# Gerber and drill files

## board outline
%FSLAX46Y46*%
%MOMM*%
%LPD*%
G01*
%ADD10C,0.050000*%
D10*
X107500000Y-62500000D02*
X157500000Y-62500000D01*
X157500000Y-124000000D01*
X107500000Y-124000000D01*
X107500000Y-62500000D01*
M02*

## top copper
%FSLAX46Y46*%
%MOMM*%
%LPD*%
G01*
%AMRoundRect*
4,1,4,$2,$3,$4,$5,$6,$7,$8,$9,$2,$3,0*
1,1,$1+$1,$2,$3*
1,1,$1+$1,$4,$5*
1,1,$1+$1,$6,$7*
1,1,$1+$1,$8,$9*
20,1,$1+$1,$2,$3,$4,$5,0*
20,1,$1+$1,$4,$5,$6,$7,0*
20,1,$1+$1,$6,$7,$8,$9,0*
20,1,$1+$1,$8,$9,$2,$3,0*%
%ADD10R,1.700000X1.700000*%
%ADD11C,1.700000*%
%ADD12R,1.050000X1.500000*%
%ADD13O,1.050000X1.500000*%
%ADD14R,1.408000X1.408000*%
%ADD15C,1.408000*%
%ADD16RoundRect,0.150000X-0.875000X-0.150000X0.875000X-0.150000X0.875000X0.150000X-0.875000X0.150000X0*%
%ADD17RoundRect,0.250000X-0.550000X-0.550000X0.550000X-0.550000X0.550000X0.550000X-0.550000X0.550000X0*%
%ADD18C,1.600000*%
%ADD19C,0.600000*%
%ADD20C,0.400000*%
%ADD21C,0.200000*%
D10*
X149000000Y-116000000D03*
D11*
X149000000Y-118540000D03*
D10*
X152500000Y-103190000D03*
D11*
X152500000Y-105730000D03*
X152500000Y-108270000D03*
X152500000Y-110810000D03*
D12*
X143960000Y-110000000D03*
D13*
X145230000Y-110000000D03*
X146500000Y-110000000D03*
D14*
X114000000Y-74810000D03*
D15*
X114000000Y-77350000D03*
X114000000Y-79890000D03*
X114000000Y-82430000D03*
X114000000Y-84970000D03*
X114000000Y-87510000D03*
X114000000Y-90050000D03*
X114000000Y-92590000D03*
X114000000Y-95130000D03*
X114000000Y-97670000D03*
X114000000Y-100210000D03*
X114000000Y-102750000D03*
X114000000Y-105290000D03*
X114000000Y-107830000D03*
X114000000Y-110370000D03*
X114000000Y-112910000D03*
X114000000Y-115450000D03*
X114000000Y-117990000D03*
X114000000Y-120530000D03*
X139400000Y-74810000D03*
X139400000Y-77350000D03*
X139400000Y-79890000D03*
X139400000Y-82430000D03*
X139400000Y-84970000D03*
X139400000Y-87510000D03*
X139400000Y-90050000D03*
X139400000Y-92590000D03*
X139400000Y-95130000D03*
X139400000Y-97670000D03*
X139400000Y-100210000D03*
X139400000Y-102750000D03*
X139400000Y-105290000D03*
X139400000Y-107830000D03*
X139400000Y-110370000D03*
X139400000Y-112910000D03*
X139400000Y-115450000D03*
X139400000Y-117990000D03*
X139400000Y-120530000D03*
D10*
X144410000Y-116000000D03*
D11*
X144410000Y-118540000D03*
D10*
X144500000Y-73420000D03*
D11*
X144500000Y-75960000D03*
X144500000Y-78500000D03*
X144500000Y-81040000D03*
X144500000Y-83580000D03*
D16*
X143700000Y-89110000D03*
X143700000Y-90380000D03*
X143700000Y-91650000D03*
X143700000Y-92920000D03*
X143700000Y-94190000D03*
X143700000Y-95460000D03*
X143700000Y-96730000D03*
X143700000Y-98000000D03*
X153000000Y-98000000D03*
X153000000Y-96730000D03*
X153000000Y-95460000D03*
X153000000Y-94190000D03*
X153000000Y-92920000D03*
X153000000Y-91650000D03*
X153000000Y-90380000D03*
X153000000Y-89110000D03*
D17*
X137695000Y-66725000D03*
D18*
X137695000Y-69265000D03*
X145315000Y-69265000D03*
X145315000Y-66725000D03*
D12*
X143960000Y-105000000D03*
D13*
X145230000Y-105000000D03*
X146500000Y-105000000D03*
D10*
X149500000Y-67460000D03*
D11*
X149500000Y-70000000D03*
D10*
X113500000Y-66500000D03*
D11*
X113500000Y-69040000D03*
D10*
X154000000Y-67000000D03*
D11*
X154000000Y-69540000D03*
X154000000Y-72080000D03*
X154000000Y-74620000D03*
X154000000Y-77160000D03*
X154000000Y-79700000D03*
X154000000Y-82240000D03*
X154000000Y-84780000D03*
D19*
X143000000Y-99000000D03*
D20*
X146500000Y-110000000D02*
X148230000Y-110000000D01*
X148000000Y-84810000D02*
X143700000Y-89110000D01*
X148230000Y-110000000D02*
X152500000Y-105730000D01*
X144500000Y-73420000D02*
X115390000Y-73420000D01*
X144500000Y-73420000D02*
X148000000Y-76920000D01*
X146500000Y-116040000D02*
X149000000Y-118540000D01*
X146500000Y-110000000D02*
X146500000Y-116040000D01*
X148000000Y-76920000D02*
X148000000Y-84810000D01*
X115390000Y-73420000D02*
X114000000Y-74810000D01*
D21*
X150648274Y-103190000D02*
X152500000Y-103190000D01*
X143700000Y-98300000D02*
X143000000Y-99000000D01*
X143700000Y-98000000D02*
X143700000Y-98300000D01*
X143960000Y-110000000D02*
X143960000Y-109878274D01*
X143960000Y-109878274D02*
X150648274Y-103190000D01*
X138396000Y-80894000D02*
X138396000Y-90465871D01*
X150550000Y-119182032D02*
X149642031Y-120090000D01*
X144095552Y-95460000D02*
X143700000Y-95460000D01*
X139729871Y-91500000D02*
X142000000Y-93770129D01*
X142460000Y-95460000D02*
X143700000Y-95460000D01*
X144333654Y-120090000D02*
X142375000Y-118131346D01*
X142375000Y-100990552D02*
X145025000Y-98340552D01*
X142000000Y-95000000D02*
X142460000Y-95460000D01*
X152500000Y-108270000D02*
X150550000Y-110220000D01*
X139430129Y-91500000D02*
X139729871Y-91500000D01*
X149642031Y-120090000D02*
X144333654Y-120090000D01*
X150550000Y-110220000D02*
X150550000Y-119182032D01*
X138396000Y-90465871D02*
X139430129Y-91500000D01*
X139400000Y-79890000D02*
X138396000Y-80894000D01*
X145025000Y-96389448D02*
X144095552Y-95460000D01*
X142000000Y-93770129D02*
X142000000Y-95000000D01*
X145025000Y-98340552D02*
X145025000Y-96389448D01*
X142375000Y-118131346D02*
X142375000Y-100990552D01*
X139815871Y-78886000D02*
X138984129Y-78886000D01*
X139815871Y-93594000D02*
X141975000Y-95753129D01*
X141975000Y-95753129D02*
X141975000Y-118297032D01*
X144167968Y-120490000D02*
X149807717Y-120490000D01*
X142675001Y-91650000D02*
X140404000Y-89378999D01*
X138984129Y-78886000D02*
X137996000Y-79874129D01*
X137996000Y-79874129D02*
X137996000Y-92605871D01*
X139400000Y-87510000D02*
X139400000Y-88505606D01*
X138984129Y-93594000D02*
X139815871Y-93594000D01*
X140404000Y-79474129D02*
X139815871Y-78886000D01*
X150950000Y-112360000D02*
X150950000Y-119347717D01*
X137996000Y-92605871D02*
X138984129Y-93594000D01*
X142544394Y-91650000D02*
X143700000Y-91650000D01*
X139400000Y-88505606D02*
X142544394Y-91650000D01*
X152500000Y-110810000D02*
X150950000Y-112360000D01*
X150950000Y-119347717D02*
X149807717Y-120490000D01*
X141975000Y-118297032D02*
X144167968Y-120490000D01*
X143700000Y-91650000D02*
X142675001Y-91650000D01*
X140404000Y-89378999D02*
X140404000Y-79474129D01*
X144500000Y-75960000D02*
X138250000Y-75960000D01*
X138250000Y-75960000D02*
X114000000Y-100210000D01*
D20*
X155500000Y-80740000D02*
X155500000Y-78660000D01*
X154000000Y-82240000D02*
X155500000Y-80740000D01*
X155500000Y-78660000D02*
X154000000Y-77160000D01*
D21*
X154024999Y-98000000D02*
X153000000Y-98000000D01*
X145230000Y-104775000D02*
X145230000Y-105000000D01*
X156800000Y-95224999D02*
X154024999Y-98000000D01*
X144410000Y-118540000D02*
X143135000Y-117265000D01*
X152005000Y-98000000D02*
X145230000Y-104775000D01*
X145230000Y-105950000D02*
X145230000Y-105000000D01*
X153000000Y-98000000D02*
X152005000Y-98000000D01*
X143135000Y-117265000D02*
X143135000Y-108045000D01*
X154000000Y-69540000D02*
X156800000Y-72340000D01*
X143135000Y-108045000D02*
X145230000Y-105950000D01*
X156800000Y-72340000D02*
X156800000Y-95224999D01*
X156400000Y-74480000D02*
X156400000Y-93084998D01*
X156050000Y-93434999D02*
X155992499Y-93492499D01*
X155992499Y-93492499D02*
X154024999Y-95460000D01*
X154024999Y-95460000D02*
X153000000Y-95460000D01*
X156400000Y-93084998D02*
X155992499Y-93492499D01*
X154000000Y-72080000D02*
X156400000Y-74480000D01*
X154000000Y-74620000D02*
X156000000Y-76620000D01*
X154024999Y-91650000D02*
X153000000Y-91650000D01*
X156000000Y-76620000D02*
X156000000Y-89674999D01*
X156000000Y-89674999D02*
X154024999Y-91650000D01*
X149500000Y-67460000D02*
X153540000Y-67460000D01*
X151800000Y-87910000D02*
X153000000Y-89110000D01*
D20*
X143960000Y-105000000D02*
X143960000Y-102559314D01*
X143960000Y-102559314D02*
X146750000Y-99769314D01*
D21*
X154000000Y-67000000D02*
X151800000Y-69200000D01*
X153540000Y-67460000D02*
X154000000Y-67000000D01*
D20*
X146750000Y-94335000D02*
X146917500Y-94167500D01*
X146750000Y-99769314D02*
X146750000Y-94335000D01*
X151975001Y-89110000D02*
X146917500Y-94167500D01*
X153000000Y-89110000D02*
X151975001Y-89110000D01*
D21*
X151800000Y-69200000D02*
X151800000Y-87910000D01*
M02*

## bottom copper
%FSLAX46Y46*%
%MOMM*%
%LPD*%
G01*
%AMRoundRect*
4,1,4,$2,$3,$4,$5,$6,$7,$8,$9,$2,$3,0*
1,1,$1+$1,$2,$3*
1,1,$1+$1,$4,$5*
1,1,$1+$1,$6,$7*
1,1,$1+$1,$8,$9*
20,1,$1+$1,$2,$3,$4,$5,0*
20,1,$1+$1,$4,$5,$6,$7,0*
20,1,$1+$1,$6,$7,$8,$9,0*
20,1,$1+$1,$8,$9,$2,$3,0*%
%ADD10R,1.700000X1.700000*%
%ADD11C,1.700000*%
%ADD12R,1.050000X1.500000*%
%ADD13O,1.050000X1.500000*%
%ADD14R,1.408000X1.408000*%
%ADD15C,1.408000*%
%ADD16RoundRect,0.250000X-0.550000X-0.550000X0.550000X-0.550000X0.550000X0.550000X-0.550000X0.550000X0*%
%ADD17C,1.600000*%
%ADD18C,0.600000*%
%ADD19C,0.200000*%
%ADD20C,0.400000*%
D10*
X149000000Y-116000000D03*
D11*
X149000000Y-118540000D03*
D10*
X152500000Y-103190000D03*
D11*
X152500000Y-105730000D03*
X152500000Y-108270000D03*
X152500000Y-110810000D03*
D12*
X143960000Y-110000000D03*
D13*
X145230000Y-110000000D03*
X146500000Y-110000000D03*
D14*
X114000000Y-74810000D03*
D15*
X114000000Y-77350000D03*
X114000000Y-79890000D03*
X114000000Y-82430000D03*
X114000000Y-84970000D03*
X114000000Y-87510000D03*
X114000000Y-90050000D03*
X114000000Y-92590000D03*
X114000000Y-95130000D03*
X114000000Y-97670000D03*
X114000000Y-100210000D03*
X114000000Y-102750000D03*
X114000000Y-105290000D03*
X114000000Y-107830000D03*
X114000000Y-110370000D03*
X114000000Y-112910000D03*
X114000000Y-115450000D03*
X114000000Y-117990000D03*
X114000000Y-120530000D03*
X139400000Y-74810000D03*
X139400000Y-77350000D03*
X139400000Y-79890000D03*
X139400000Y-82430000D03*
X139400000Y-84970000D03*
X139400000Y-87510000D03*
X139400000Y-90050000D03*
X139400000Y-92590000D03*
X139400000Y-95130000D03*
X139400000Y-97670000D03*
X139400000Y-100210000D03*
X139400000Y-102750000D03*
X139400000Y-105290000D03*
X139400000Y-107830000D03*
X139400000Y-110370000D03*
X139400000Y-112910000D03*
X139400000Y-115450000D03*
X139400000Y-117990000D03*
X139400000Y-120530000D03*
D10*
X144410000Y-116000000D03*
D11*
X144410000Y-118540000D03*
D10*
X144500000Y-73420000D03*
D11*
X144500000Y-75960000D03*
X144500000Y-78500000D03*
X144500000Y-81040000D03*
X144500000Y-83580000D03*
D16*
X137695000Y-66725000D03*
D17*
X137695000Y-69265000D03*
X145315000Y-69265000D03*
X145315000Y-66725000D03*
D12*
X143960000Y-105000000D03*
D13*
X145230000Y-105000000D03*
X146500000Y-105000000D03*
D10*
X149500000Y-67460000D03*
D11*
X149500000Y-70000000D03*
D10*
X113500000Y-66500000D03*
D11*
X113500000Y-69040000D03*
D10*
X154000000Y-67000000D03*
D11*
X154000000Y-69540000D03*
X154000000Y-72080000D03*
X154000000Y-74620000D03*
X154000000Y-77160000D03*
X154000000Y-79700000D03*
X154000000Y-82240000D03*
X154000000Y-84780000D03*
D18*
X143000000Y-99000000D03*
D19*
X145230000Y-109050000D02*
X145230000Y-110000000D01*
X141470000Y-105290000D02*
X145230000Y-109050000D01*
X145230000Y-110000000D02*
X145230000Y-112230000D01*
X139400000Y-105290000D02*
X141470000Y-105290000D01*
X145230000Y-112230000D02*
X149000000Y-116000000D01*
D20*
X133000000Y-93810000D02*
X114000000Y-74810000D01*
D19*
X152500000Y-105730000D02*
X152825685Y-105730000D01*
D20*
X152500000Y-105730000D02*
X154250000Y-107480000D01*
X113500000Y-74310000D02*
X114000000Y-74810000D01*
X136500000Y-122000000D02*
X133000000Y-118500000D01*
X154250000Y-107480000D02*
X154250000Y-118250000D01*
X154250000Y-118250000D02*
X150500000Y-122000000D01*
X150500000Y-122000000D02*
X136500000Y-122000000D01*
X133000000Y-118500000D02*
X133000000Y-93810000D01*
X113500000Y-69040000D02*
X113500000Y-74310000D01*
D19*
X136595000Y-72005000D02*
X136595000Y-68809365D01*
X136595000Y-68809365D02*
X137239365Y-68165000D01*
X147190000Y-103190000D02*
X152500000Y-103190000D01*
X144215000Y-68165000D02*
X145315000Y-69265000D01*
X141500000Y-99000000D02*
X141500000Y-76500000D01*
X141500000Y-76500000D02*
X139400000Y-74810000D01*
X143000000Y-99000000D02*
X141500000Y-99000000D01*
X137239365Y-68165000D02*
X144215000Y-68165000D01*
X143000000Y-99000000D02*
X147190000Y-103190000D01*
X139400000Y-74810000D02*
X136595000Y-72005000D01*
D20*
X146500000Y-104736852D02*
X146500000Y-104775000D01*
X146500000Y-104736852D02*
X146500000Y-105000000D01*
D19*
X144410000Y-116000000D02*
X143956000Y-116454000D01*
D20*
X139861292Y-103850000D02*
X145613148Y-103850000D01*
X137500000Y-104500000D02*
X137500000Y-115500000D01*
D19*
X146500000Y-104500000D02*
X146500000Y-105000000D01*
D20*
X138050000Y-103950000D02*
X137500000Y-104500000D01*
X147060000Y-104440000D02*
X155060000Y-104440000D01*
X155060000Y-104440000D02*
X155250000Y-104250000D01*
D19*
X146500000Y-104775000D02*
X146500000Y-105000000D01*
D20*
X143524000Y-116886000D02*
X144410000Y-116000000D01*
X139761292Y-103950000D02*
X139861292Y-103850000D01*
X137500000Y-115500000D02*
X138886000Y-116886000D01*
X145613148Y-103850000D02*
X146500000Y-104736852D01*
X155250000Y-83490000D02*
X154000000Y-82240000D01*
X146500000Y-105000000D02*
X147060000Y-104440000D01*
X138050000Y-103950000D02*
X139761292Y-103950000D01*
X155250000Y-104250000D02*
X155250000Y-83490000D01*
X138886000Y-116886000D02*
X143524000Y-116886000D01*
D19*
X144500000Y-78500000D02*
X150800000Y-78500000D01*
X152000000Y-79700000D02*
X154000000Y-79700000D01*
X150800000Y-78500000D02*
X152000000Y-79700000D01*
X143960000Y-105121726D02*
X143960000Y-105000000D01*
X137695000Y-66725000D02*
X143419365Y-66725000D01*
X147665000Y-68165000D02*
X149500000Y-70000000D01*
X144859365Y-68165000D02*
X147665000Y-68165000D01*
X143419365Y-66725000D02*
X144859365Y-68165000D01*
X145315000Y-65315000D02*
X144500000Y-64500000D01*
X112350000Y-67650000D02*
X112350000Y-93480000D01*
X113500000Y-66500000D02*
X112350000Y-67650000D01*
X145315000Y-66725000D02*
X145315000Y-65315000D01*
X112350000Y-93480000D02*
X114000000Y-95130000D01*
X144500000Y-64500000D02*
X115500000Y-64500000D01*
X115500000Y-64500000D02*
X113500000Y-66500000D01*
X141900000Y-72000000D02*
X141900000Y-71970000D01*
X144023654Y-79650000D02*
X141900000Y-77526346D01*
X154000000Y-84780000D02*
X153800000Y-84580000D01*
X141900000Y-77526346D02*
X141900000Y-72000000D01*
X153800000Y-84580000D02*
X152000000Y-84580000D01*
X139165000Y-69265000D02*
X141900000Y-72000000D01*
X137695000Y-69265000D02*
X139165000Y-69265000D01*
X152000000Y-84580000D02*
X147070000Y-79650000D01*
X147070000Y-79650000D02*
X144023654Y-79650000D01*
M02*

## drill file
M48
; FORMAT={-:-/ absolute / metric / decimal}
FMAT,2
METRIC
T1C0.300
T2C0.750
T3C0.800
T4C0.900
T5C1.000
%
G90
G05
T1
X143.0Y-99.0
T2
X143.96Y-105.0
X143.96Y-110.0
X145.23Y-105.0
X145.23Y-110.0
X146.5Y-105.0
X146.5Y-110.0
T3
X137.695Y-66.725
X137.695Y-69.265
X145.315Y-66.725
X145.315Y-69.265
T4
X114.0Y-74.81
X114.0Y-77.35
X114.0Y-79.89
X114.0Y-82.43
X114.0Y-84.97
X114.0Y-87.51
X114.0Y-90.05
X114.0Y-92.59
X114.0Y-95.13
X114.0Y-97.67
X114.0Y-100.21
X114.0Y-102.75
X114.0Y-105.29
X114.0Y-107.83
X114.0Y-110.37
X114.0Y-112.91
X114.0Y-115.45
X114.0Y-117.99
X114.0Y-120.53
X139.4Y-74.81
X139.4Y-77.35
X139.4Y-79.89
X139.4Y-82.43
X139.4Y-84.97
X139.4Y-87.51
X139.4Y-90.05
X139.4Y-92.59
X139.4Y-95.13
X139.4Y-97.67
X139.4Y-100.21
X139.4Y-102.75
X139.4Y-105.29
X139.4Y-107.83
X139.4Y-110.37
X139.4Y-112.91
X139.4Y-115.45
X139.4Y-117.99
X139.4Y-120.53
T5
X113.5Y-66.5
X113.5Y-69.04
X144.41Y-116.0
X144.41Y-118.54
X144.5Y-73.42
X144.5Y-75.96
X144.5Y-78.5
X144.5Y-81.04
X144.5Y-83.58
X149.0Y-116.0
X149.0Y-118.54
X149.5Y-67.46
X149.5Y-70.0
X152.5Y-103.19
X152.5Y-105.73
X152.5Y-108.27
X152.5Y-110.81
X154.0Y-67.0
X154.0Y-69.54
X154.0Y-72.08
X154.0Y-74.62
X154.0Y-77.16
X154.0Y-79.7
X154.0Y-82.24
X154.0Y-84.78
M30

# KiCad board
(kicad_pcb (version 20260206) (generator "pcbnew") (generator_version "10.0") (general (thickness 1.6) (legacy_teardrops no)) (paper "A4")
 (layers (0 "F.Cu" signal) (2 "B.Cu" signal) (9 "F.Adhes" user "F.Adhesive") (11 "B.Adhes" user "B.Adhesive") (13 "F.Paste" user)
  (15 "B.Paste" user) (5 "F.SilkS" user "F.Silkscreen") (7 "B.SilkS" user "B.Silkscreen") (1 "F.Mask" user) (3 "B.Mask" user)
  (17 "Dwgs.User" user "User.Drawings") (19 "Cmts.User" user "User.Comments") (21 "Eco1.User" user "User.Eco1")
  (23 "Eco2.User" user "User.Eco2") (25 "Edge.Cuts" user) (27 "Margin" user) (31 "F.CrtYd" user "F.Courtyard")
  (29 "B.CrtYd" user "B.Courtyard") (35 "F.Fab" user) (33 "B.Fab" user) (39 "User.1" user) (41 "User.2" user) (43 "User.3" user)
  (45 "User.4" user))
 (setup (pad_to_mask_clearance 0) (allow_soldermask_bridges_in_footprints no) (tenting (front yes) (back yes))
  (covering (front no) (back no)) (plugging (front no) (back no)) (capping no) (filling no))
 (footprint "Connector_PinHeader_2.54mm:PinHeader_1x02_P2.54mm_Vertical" (layer "F.Cu") (at 149 116)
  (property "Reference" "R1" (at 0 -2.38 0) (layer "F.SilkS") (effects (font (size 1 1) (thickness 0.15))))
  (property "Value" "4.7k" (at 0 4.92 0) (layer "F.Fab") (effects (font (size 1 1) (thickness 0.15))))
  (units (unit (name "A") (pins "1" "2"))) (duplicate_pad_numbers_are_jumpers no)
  (pad "1" thru_hole rect (at 0 0) (size 1.7 1.7) (drill 1) (layers "*.Cu" "*.Mask") (remove_unused_layers no) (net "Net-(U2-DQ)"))
  (pad "2" thru_hole circle (at 0 2.54) (size 1.7 1.7) (drill 1) (layers "*.Cu" "*.Mask") (remove_unused_layers no) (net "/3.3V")))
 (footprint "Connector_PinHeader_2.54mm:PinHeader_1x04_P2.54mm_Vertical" (layer "F.Cu") (at 152.5 103.19)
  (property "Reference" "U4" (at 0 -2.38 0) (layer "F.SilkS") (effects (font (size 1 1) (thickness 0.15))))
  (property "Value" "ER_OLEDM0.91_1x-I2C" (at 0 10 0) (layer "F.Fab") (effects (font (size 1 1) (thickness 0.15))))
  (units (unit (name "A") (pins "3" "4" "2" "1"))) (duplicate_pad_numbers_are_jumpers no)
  (pad "1" thru_hole rect (at 0 0) (size 1.7 1.7) (drill 1) (layers "*.Cu" "*.Mask") (remove_unused_layers no) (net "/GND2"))
  (pad "2" thru_hole circle (at 0 2.54) (size 1.7 1.7) (drill 1) (layers "*.Cu" "*.Mask") (remove_unused_layers no) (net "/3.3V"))
  (pad "3" thru_hole circle (at 0 5.08) (size 1.7 1.7) (drill 1) (layers "*.Cu" "*.Mask") (remove_unused_layers no) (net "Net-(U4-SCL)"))
  (pad "4" thru_hole circle (at 0 7.62) (size 1.7 1.7) (drill 1) (layers "*.Cu" "*.Mask") (remove_unused_layers no) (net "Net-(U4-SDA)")))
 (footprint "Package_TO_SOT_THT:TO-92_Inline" (layer "F.Cu") (at 143.96 110)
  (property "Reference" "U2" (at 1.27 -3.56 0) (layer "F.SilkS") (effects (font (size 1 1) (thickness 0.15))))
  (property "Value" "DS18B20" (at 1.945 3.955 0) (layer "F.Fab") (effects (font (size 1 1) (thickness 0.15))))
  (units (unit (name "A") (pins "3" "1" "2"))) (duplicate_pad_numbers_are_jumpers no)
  (pad "1" thru_hole rect (at 0 0) (size 1.05 1.5) (drill 0.75) (layers "*.Cu" "*.Mask") (remove_unused_layers no) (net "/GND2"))
  (pad "2" thru_hole oval (at 1.27 0) (size 1.05 1.5) (drill 0.75) (layers "*.Cu" "*.Mask") (remove_unused_layers no) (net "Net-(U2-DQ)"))
  (pad "3" thru_hole oval (at 2.54 0) (size 1.05 1.5) (drill 0.75) (layers "*.Cu" "*.Mask") (remove_unused_layers no) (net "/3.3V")))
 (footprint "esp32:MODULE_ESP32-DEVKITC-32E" (layer "F.Cu") (at 126.7 97.645)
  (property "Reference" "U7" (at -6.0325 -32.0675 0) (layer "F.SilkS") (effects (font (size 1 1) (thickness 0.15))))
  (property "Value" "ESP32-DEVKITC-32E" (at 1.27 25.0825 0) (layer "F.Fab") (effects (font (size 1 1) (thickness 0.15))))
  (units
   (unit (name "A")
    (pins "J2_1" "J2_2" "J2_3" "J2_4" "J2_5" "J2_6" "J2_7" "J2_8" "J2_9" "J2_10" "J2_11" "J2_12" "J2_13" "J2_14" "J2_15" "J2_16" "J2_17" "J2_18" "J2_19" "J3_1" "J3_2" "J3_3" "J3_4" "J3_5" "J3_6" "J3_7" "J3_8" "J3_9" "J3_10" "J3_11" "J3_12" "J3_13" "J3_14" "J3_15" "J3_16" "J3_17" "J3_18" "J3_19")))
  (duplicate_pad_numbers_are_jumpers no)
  (pad "J2_1" thru_hole rect (at -12.7 -22.835) (size 1.408 1.408) (drill 0.9) (layers "*.Cu" "*.Mask") (remove_unused_layers no)
   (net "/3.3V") (solder_mask_margin 0.102))
  (pad "J2_2" thru_hole circle (at -12.7 -20.295) (size 1.408 1.408) (drill 0.9) (layers "*.Cu" "*.Mask") (remove_unused_layers no)
   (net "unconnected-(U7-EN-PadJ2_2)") (solder_mask_margin 0.102))
  (pad "J2_3" thru_hole circle (at -12.7 -17.755) (size 1.408 1.408) (drill 0.9) (layers "*.Cu" "*.Mask") (remove_unused_layers no)
   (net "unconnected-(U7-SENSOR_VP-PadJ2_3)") (solder_mask_margin 0.102))
  (pad "J2_4" thru_hole circle (at -12.7 -15.215) (size 1.408 1.408) (drill 0.9) (layers "*.Cu" "*.Mask") (remove_unused_layers no)
   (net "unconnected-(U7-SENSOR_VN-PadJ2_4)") (solder_mask_margin 0.102))
  (pad "J2_5" thru_hole circle (at -12.7 -12.675) (size 1.408 1.408) (drill 0.9) (layers "*.Cu" "*.Mask") (remove_unused_layers no)
   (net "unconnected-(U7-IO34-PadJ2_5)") (solder_mask_margin 0.102))
  (pad "J2_6" thru_hole circle (at -12.7 -10.135) (size 1.408 1.408) (drill 0.9) (layers "*.Cu" "*.Mask") (remove_unused_layers no)
   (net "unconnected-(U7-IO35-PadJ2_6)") (solder_mask_margin 0.102))
  (pad "J2_7" thru_hole circle (at -12.7 -7.595) (size 1.408 1.408) (drill 0.9) (layers "*.Cu" "*.Mask") (remove_unused_layers no)
   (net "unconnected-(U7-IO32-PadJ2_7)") (solder_mask_margin 0.102))
  (pad "J2_8" thru_hole circle (at -12.7 -5.055) (size 1.408 1.408) (drill 0.9) (layers "*.Cu" "*.Mask") (remove_unused_layers no)
   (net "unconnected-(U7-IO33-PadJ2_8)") (solder_mask_margin 0.102))
  (pad "J2_9" thru_hole circle (at -12.7 -2.515) (size 1.408 1.408) (drill 0.9) (layers "*.Cu" "*.Mask") (remove_unused_layers no)
   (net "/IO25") (solder_mask_margin 0.102))
  (pad "J2_10" thru_hole circle (at -12.7 0.025) (size 1.408 1.408) (drill 0.9) (layers "*.Cu" "*.Mask") (remove_unused_layers no)
   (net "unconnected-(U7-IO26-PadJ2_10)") (solder_mask_margin 0.102))
  (pad "J2_11" thru_hole circle (at -12.7 2.565) (size 1.408 1.408) (drill 0.9) (layers "*.Cu" "*.Mask") (remove_unused_layers no)
   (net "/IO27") (solder_mask_margin 0.102))
  (pad "J2_12" thru_hole circle (at -12.7 5.105) (size 1.408 1.408) (drill 0.9) (layers "*.Cu" "*.Mask") (remove_unused_layers no)
   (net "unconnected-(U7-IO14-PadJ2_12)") (solder_mask_margin 0.102))
  (pad "J2_13" thru_hole circle (at -12.7 7.645) (size 1.408 1.408) (drill 0.9) (layers "*.Cu" "*.Mask") (remove_unused_layers no)
   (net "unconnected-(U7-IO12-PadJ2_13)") (solder_mask_margin 0.102))
  (pad "J2_14" thru_hole circle (at -12.7 10.185) (size 1.408 1.408) (drill 0.9) (layers "*.Cu" "*.Mask") (remove_unused_layers no)
   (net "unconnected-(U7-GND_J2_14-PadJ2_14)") (solder_mask_margin 0.102))
  (pad "J2_15" thru_hole circle (at -12.7 12.725) (size 1.408 1.408) (drill 0.9) (layers "*.Cu" "*.Mask") (remove_unused_layers no)
   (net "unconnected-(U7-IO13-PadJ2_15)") (solder_mask_margin 0.102))
  (pad "J2_16" thru_hole circle (at -12.7 15.265) (size 1.408 1.408) (drill 0.9) (layers "*.Cu" "*.Mask") (remove_unused_layers no)
   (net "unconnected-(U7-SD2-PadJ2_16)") (solder_mask_margin 0.102))
  (pad "J2_17" thru_hole circle (at -12.7 17.805) (size 1.408 1.408) (drill 0.9) (layers "*.Cu" "*.Mask") (remove_unused_layers no)
   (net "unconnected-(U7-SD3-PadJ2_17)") (solder_mask_margin 0.102))
  (pad "J2_18" thru_hole circle (at -12.7 20.345) (size 1.408 1.408) (drill 0.9) (layers "*.Cu" "*.Mask") (remove_unused_layers no)
   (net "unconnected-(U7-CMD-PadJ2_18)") (solder_mask_margin 0.102))
  (pad "J2_19" thru_hole circle (at -12.7 22.885) (size 1.408 1.408) (drill 0.9) (layers "*.Cu" "*.Mask") (remove_unused_layers no)
   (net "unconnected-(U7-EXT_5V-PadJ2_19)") (solder_mask_margin 0.102))
  (pad "J3_1" thru_hole circle (at 12.7 -22.835) (size 1.408 1.408) (drill 0.9) (layers "*.Cu" "*.Mask") (remove_unused_layers no)
   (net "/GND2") (solder_mask_margin 0.102))
  (pad "J3_2" thru_hole circle (at 12.7 -20.295) (size 1.408 1.408) (drill 0.9) (layers "*.Cu" "*.Mask") (remove_unused_layers no)
   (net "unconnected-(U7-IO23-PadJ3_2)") (solder_mask_margin 0.102))
  (pad "J3_3" thru_hole circle (at 12.7 -17.755) (size 1.408 1.408) (drill 0.9) (layers "*.Cu" "*.Mask") (remove_unused_layers no)
   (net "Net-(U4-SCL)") (solder_mask_margin 0.102))
  (pad "J3_4" thru_hole circle (at 12.7 -15.215) (size 1.408 1.408) (drill 0.9) (layers "*.Cu" "*.Mask") (remove_unused_layers no)
   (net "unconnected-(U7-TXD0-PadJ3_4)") (solder_mask_margin 0.102))
  (pad "J3_5" thru_hole circle (at 12.7 -12.675) (size 1.408 1.408) (drill 0.9) (layers "*.Cu" "*.Mask") (remove_unused_layers no)
   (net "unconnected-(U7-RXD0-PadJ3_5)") (solder_mask_margin 0.102))
  (pad "J3_6" thru_hole circle (at 12.7 -10.135) (size 1.408 1.408) (drill 0.9) (layers "*.Cu" "*.Mask") (remove_unused_layers no)
   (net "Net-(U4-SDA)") (solder_mask_margin 0.102))
  (pad "J3_7" thru_hole circle (at 12.7 -7.595) (size 1.408 1.408) (drill 0.9) (layers "*.Cu" "*.Mask") (remove_unused_layers no)
   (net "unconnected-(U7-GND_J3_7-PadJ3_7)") (solder_mask_margin 0.102))
  (pad "J3_8" thru_hole circle (at 12.7 -5.055) (size 1.408 1.408) (drill 0.9) (layers "*.Cu" "*.Mask") (remove_unused_layers no)
   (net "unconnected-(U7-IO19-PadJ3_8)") (solder_mask_margin 0.102))
  (pad "J3_9" thru_hole circle (at 12.7 -2.515) (size 1.408 1.408) (drill 0.9) (layers "*.Cu" "*.Mask") (remove_unused_layers no)
   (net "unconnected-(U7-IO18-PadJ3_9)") (solder_mask_margin 0.102))
  (pad "J3_10" thru_hole circle (at 12.7 0.025) (size 1.408 1.408) (drill 0.9) (layers "*.Cu" "*.Mask") (remove_unused_layers no)
   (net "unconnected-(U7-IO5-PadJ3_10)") (solder_mask_margin 0.102))
  (pad "J3_11" thru_hole circle (at 12.7 2.565) (size 1.408 1.408) (drill 0.9) (layers "*.Cu" "*.Mask") (remove_unused_layers no)
   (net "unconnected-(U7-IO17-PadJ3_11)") (solder_mask_margin 0.102))
  (pad "J3_12" thru_hole circle (at 12.7 5.105) (size 1.408 1.408) (drill 0.9) (layers "*.Cu" "*.Mask") (remove_unused_layers no)
   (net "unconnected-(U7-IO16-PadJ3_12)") (solder_mask_margin 0.102))
  (pad "J3_13" thru_hole circle (at 12.7 7.645) (size 1.408 1.408) (drill 0.9) (layers "*.Cu" "*.Mask") (remove_unused_layers no)
   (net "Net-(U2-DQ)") (solder_mask_margin 0.102))
  (pad "J3_14" thru_hole circle (at 12.7 10.185) (size 1.408 1.408) (drill 0.9) (layers "*.Cu" "*.Mask") (remove_unused_layers no)
   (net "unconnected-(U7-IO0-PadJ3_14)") (solder_mask_margin 0.102))
  (pad "J3_15" thru_hole circle (at 12.7 12.725) (size 1.408 1.408) (drill 0.9) (layers "*.Cu" "*.Mask") (remove_unused_layers no)
   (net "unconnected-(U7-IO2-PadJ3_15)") (solder_mask_margin 0.102))
  (pad "J3_16" thru_hole circle (at 12.7 15.265) (size 1.408 1.408) (drill 0.9) (layers "*.Cu" "*.Mask") (remove_unused_layers no)
   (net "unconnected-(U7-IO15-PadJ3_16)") (solder_mask_margin 0.102))
  (pad "J3_17" thru_hole circle (at 12.7 17.805) (size 1.408 1.408) (drill 0.9) (layers "*.Cu" "*.Mask") (remove_unused_layers no)
   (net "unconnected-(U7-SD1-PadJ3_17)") (solder_mask_margin 0.102))
  (pad "J3_18" thru_hole circle (at 12.7 20.345) (size 1.408 1.408) (drill 0.9) (layers "*.Cu" "*.Mask") (remove_unused_layers no)
   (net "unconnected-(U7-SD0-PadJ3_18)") (solder_mask_margin 0.102))
  (pad "J3_19" thru_hole circle (at 12.7 22.885) (size 1.408 1.408) (drill 0.9) (layers "*.Cu" "*.Mask") (remove_unused_layers no)
   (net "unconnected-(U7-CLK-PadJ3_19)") (solder_mask_margin 0.102)))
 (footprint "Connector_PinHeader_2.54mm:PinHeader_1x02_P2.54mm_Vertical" (layer "F.Cu") (at 144.41 116)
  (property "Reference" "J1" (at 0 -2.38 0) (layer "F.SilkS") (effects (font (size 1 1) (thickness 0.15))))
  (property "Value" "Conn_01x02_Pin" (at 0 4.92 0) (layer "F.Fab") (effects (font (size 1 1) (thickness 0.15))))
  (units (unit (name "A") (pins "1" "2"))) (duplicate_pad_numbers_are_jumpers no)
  (pad "1" thru_hole rect (at 0 0) (size 1.7 1.7) (drill 1) (layers "*.Cu" "*.Mask") (remove_unused_layers no) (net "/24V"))
  (pad "2" thru_hole circle (at 0 2.54) (size 1.7 1.7) (drill 1) (layers "*.Cu" "*.Mask") (remove_unused_layers no) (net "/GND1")))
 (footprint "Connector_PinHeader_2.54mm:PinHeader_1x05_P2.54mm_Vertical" (layer "F.Cu") (at 144.5 73.42)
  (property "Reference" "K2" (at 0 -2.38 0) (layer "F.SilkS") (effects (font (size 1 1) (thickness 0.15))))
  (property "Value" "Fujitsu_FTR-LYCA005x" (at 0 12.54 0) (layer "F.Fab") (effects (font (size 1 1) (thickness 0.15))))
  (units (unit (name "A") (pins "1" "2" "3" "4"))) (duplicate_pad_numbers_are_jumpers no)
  (pad "1" thru_hole rect (at 0 0) (size 1.7 1.7) (drill 1) (layers "*.Cu" "*.Mask") (remove_unused_layers no) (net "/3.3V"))
  (pad "2" thru_hole circle (at 0 2.54) (size 1.7 1.7) (drill 1) (layers "*.Cu" "*.Mask") (remove_unused_layers no) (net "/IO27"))
  (pad "3" thru_hole circle (at 0 5.08) (size 1.7 1.7) (drill 1) (layers "*.Cu" "*.Mask") (remove_unused_layers no) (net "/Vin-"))
  (pad "4" thru_hole circle (at 0 7.62) (size 1.7 1.7) (drill 1) (layers "*.Cu" "*.Mask") (remove_unused_layers no) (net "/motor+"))
  (pad "5" thru_hole circle (at 0 10.16) (size 1.7 1.7) (drill 1) (layers "*.Cu" "*.Mask") (remove_unused_layers no)))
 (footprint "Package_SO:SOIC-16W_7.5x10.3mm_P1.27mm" (layer "F.Cu") (at 148.35 93.555)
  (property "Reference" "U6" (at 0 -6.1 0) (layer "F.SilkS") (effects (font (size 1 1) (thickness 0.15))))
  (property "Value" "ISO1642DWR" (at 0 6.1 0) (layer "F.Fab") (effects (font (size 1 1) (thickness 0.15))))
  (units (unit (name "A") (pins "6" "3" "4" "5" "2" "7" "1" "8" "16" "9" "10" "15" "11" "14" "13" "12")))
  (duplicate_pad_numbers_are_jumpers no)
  (pad "1" smd roundrect (at -4.65 -4.445) (size 2.05 0.6) (layers "F.Cu" "F.Mask" "F.Paste") (roundrect_rratio 0.25) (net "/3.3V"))
  (pad "2" smd roundrect (at -4.65 -3.175) (size 2.05 0.6) (layers "F.Cu" "F.Mask" "F.Paste") (roundrect_rratio 0.25)
   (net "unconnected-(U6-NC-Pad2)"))
  (pad "3" smd roundrect (at -4.65 -1.905) (size 2.05 0.6) (layers "F.Cu" "F.Mask" "F.Paste") (roundrect_rratio 0.25) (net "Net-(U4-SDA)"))
  (pad "4" smd roundrect (at -4.65 -0.635) (size 2.05 0.6) (layers "F.Cu" "F.Mask" "F.Paste") (roundrect_rratio 0.25)
   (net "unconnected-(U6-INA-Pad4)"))
  (pad "5" smd roundrect (at -4.65 0.635) (size 2.05 0.6) (layers "F.Cu" "F.Mask" "F.Paste") (roundrect_rratio 0.25)
   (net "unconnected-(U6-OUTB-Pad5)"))
  (pad "6" smd roundrect (at -4.65 1.905) (size 2.05 0.6) (layers "F.Cu" "F.Mask" "F.Paste") (roundrect_rratio 0.25) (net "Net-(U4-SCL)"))
  (pad "7" smd roundrect (at -4.65 3.175) (size 2.05 0.6) (layers "F.Cu" "F.Mask" "F.Paste") (roundrect_rratio 0.25)
   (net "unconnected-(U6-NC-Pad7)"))
  (pad "8" smd roundrect (at -4.65 4.445) (size 2.05 0.6) (layers "F.Cu" "F.Mask" "F.Paste") (roundrect_rratio 0.25) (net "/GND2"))
  (pad "9" smd roundrect (at 4.65 4.445) (size 2.05 0.6) (layers "F.Cu" "F.Mask" "F.Paste") (roundrect_rratio 0.25) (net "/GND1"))
  (pad "10" smd roundrect (at 4.65 3.175) (size 2.05 0.6) (layers "F.Cu" "F.Mask" "F.Paste") (roundrect_rratio 0.25)
   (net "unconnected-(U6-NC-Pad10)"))
  (pad "11" smd roundrect (at 4.65 1.905) (size 2.05 0.6) (layers "F.Cu" "F.Mask" "F.Paste") (roundrect_rratio 0.25) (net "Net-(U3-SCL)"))
  (pad "12" smd roundrect (at 4.65 0.635) (size 2.05 0.6) (layers "F.Cu" "F.Mask" "F.Paste") (roundrect_rratio 0.25)
   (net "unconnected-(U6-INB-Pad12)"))
  (pad "13" smd roundrect (at 4.65 -0.635) (size 2.05 0.6) (layers "F.Cu" "F.Mask" "F.Paste") (roundrect_rratio 0.25)
   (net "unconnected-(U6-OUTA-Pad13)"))
  (pad "14" smd roundrect (at 4.65 -1.905) (size 2.05 0.6) (layers "F.Cu" "F.Mask" "F.Paste") (roundrect_rratio 0.25) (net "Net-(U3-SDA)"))
  (pad "15" smd roundrect (at 4.65 -3.175) (size 2.05 0.6) (layers "F.Cu" "F.Mask" "F.Paste") (roundrect_rratio 0.25)
   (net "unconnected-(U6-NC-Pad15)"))
  (pad "16" smd roundrect (at 4.65 -4.445) (size 2.05 0.6) (layers "F.Cu" "F.Mask" "F.Paste") (roundrect_rratio 0.25) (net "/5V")))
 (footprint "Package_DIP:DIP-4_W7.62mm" (layer "F.Cu") (at 137.695 66.725)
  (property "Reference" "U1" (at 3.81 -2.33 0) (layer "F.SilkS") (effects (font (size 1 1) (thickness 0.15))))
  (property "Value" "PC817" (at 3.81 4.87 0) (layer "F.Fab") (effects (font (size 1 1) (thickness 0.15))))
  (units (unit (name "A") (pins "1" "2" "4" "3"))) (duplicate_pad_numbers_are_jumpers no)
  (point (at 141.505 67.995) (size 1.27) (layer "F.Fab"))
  (pad "1" thru_hole roundrect (at 0 0) (size 1.6 1.6) (drill 0.8) (layers "*.Cu" "*.Mask") (remove_unused_layers no)
   (roundrect_rratio 0.15625) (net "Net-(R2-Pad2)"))
  (pad "2" thru_hole circle (at 0 2.54) (size 1.6 1.6) (drill 0.8) (layers "*.Cu" "*.Mask") (remove_unused_layers no) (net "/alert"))
  (pad "3" thru_hole circle (at 7.62 2.54) (size 1.6 1.6) (drill 0.8) (layers "*.Cu" "*.Mask") (remove_unused_layers no) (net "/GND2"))
  (pad "4" thru_hole circle (at 7.62 0) (size 1.6 1.6) (drill 0.8) (layers "*.Cu" "*.Mask") (remove_unused_layers no) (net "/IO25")))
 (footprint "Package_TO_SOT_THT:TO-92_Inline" (layer "F.Cu") (at 143.96 105)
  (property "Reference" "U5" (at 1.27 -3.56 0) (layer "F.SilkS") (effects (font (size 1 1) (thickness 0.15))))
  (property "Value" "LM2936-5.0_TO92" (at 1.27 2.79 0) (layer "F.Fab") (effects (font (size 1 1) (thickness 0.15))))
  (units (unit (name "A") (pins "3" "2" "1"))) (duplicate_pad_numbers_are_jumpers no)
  (pad "1" thru_hole rect (at 0 0) (size 1.05 1.5) (drill 0.75) (layers "*.Cu" "*.Mask") (remove_unused_layers no) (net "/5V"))
  (pad "2" thru_hole oval (at 1.27 0) (size 1.05 1.5) (drill 0.75) (layers "*.Cu" "*.Mask") (remove_unused_layers no) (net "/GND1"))
  (pad "3" thru_hole oval (at 2.54 0) (size 1.05 1.5) (drill 0.75) (layers "*.Cu" "*.Mask") (remove_unused_layers no) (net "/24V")))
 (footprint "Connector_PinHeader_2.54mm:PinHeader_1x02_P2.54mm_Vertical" (layer "F.Cu") (at 149.5 67.46)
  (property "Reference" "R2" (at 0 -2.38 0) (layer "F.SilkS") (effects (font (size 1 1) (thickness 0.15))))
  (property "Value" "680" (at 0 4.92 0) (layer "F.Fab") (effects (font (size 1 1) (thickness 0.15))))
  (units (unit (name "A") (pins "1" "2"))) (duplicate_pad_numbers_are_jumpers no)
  (pad "1" thru_hole rect (at 0 0) (size 1.7 1.7) (drill 1) (layers "*.Cu" "*.Mask") (remove_unused_layers no) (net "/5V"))
  (pad "2" thru_hole circle (at 0 2.54) (size 1.7 1.7) (drill 1) (layers "*.Cu" "*.Mask") (remove_unused_layers no) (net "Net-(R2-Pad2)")))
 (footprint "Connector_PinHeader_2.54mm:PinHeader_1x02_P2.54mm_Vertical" (layer "F.Cu") (at 113.5 66.5)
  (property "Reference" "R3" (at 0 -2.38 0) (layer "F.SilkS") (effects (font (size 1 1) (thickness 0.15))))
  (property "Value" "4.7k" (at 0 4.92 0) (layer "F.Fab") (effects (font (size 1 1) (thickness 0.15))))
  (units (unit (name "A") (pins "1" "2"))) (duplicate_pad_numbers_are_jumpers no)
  (pad "1" thru_hole rect (at 0 0) (size 1.7 1.7) (drill 1) (layers "*.Cu" "*.Mask") (remove_unused_layers no) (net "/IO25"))
  (pad "2" thru_hole circle (at 0 2.54) (size 1.7 1.7) (drill 1) (layers "*.Cu" "*.Mask") (remove_unused_layers no) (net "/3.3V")))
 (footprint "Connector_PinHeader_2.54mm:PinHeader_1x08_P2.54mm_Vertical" (layer "F.Cu") (at 154 67)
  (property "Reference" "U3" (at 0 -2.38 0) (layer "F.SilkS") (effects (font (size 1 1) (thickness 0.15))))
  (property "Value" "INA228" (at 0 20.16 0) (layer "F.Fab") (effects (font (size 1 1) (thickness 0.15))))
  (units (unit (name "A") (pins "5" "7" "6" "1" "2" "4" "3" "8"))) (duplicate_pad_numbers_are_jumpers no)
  (pad "1" thru_hole rect (at 0 0) (size 1.7 1.7) (drill 1) (layers "*.Cu" "*.Mask") (remove_unused_layers no) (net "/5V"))
  (pad "2" thru_hole circle (at 0 2.54) (size 1.7 1.7) (drill 1) (layers "*.Cu" "*.Mask") (remove_unused_layers no) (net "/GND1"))
  (pad "3" thru_hole circle (at 0 5.08) (size 1.7 1.7) (drill 1) (layers "*.Cu" "*.Mask") (remove_unused_layers no) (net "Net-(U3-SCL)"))
  (pad "4" thru_hole circle (at 0 7.62) (size 1.7 1.7) (drill 1) (layers "*.Cu" "*.Mask") (remove_unused_layers no) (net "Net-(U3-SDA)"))
  (pad "5" thru_hole circle (at 0 10.16) (size 1.7 1.7) (drill 1) (layers "*.Cu" "*.Mask") (remove_unused_layers no) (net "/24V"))
  (pad "6" thru_hole circle (at 0 12.7) (size 1.7 1.7) (drill 1) (layers "*.Cu" "*.Mask") (remove_unused_layers no) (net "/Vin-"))
  (pad "7" thru_hole circle (at 0 15.24) (size 1.7 1.7) (drill 1) (layers "*.Cu" "*.Mask") (remove_unused_layers no) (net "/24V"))
  (pad "8" thru_hole circle (at 0 17.78) (size 1.7 1.7) (drill 1) (layers "*.Cu" "*.Mask") (remove_unused_layers no) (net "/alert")))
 (gr_rect (start 107.5 62.5) (end 157.5 124) (stroke (width 0.05) (type default)) (fill no) (layer "Edge.Cuts"))
 (segment (start 145.23 109.05) (end 145.23 110) (width 0.2) (layer "B.Cu") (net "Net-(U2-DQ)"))
 (segment (start 141.47 105.29) (end 145.23 109.05) (width 0.2) (layer "B.Cu") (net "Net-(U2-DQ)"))
 (segment (start 145.23 110) (end 145.23 112.23) (width 0.2) (layer "B.Cu") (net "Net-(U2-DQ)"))
 (segment (start 139.4 105.29) (end 141.47 105.29) (width 0.2) (layer "B.Cu") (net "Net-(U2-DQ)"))
 (segment (start 145.23 112.23) (end 149 116) (width 0.2) (layer "B.Cu") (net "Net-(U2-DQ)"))
 (segment (start 146.5 110) (end 148.23 110) (width 0.4) (layer "F.Cu") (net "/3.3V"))
 (segment (start 148 84.81) (end 143.7 89.11) (width 0.4) (layer "F.Cu") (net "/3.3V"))
 (segment (start 148.23 110) (end 152.5 105.73) (width 0.4) (layer "F.Cu") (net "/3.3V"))
 (segment (start 144.5 73.42) (end 115.39 73.42) (width 0.4) (layer "F.Cu") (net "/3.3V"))
 (segment (start 144.5 73.42) (end 148 76.92) (width 0.4) (layer "F.Cu") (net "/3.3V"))
 (segment (start 146.5 116.04) (end 149 118.54) (width 0.4) (layer "F.Cu") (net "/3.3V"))
 (segment (start 146.5 110) (end 146.5 116.04) (width 0.4) (layer "F.Cu") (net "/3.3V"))
 (segment (start 148 76.92) (end 148 84.81) (width 0.4) (layer "F.Cu") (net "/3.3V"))
 (segment (start 115.39 73.42) (end 114 74.81) (width 0.4) (layer "F.Cu") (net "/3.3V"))
 (segment (start 133 93.81) (end 114 74.81) (width 0.4) (layer "B.Cu") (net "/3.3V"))
 (segment (start 152.5 105.73) (end 152.825685 105.73) (width 0.2) (layer "B.Cu") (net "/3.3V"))
 (segment (start 152.5 105.73) (end 154.25 107.48) (width 0.4) (layer "B.Cu") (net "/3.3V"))
 (segment (start 113.5 74.31) (end 114 74.81) (width 0.4) (layer "B.Cu") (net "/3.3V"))
 (segment (start 136.5 122) (end 133 118.5) (width 0.4) (layer "B.Cu") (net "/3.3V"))
 (segment (start 154.25 107.48) (end 154.25 118.25) (width 0.4) (layer "B.Cu") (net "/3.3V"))
 (segment (start 154.25 118.25) (end 150.5 122) (width 0.4) (layer "B.Cu") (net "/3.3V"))
 (segment (start 150.5 122) (end 136.5 122) (width 0.4) (layer "B.Cu") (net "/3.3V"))
 (segment (start 133 118.5) (end 133 93.81) (width 0.4) (layer "B.Cu") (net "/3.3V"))
 (segment (start 113.5 69.04) (end 113.5 74.31) (width 0.4) (layer "B.Cu") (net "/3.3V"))
 (segment (start 150.648274 103.19) (end 152.5 103.19) (width 0.2) (layer "F.Cu") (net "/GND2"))
 (segment (start 143.7 98.3) (end 143 99) (width 0.2) (layer "F.Cu") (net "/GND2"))
 (segment (start 143.7 98) (end 143.7 98.3) (width 0.2) (layer "F.Cu") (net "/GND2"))
 (segment (start 143.96 110) (end 143.96 109.878274) (width 0.2) (layer "F.Cu") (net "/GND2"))
 (segment (start 143.96 109.878274) (end 150.648274 103.19) (width 0.2) (layer "F.Cu") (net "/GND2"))
 (via (at 143 99) (size 0.6) (drill 0.3) (layers "F.Cu" "B.Cu") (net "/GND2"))
 (segment (start 136.595 72.005) (end 136.595 68.809365) (width 0.2) (layer "B.Cu") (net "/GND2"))
 (segment (start 136.595 68.809365) (end 137.239365 68.165) (width 0.2) (layer "B.Cu") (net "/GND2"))
 (segment (start 147.19 103.19) (end 152.5 103.19) (width 0.2) (layer "B.Cu") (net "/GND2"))
 (segment (start 144.215 68.165) (end 145.315 69.265) (width 0.2) (layer "B.Cu") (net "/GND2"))
 (segment (start 141.5 99) (end 141.5 76.5) (width 0.2) (layer "B.Cu") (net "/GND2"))
 (segment (start 141.5 76.5) (end 139.4 74.81) (width 0.2) (layer "B.Cu") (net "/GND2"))
 (segment (start 143 99) (end 141.5 99) (width 0.2) (layer "B.Cu") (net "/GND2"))
 (segment (start 137.239365 68.165) (end 144.215 68.165) (width 0.2) (layer "B.Cu") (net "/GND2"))
 (segment (start 143 99) (end 147.19 103.19) (width 0.2) (layer "B.Cu") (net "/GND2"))
 (segment (start 139.4 74.81) (end 136.595 72.005) (width 0.2) (layer "B.Cu") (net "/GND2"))
 (segment (start 138.396 80.894) (end 138.396 90.465871) (width 0.2) (layer "F.Cu") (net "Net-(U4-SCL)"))
 (segment (start 150.55 119.182032) (end 149.642031 120.09) (width 0.2) (layer "F.Cu") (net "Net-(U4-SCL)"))
 (segment (start 144.095552 95.46) (end 143.7 95.46) (width 0.2) (layer "F.Cu") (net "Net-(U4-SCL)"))
 (segment (start 139.729871 91.5) (end 142 93.770129) (width 0.2) (layer "F.Cu") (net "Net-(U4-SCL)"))
 (segment (start 142.46 95.46) (end 143.7 95.46) (width 0.2) (layer "F.Cu") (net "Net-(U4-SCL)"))
 (segment (start 144.333654 120.09) (end 142.375 118.131346) (width 0.2) (layer "F.Cu") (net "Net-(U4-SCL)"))
 (segment (start 142.375 100.990552) (end 145.025 98.340552) (width 0.2) (layer "F.Cu") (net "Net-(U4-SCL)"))
 (segment (start 142 95) (end 142.46 95.46) (width 0.2) (layer "F.Cu") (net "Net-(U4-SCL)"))
 (segment (start 152.5 108.27) (end 150.55 110.22) (width 0.2) (layer "F.Cu") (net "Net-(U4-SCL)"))
 (segment (start 139.430129 91.5) (end 139.729871 91.5) (width 0.2) (layer "F.Cu") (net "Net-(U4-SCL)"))
 (segment (start 149.642031 120.09) (end 144.333654 120.09) (width 0.2) (layer "F.Cu") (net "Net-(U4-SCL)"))
 (segment (start 150.55 110.22) (end 150.55 119.182032) (width 0.2) (layer "F.Cu") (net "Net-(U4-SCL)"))
 (segment (start 138.396 90.465871) (end 139.430129 91.5) (width 0.2) (layer "F.Cu") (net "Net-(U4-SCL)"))
 (segment (start 139.4 79.89) (end 138.396 80.894) (width 0.2) (layer "F.Cu") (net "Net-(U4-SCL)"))
 (segment (start 145.025 96.389448) (end 144.095552 95.46) (width 0.2) (layer "F.Cu") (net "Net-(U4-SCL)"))
 (segment (start 142 93.770129) (end 142 95) (width 0.2) (layer "F.Cu") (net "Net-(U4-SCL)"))
 (segment (start 145.025 98.340552) (end 145.025 96.389448) (width 0.2) (layer "F.Cu") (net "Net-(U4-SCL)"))
 (segment (start 142.375 118.131346) (end 142.375 100.990552) (width 0.2) (layer "F.Cu") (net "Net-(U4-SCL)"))
 (segment (start 139.815871 78.886) (end 138.984129 78.886) (width 0.2) (layer "F.Cu") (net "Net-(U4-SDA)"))
 (segment (start 139.815871 93.594) (end 141.975 95.753129) (width 0.2) (layer "F.Cu") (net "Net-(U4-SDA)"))
 (segment (start 141.975 95.753129) (end 141.975 118.297032) (width 0.2) (layer "F.Cu") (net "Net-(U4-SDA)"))
 (segment (start 144.167968 120.49) (end 149.807717 120.49) (width 0.2) (layer "F.Cu") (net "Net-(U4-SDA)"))
 (segment (start 142.675001 91.65) (end 140.404 89.378999) (width 0.2) (layer "F.Cu") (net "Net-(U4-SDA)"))
 (segment (start 138.984129 78.886) (end 137.996 79.874129) (width 0.2) (layer "F.Cu") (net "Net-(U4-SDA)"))
 (segment (start 137.996 79.874129) (end 137.996 92.605871) (width 0.2) (layer "F.Cu") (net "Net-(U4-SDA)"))
 (segment (start 139.4 87.51) (end 139.4 88.505606) (width 0.2) (layer "F.Cu") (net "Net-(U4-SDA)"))
 (segment (start 138.984129 93.594) (end 139.815871 93.594) (width 0.2) (layer "F.Cu") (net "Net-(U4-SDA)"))
 (segment (start 140.404 79.474129) (end 139.815871 78.886) (width 0.2) (layer "F.Cu") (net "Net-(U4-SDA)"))
 (segment (start 150.95 112.36) (end 150.95 119.347717) (width 0.2) (layer "F.Cu") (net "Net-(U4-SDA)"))
 (segment (start 137.996 92.605871) (end 138.984129 93.594) (width 0.2) (layer "F.Cu") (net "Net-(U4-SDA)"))
 (segment (start 142.544394 91.65) (end 143.7 91.65) (width 0.2) (layer "F.Cu") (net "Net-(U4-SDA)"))
 (segment (start 139.4 88.505606) (end 142.544394 91.65) (width 0.2) (layer "F.Cu") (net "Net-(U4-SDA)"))
 (segment (start 152.5 110.81) (end 150.95 112.36) (width 0.2) (layer "F.Cu") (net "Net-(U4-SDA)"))
 (segment (start 150.95 119.347717) (end 149.807717 120.49) (width 0.2) (layer "F.Cu") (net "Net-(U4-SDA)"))
 (segment (start 141.975 118.297032) (end 144.167968 120.49) (width 0.2) (layer "F.Cu") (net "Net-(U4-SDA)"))
 (segment (start 143.7 91.65) (end 142.675001 91.65) (width 0.2) (layer "F.Cu") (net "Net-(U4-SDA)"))
 (segment (start 140.404 89.378999) (end 140.404 79.474129) (width 0.2) (layer "F.Cu") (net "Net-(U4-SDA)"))
 (segment (start 144.5 75.96) (end 138.25 75.96) (width 0.2) (layer "F.Cu") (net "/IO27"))
 (segment (start 138.25 75.96) (end 114 100.21) (width 0.2) (layer "F.Cu") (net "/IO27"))
 (segment (start 155.5 80.74) (end 155.5 78.66) (width 0.4) (layer "F.Cu") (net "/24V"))
 (segment (start 154 82.24) (end 155.5 80.74) (width 0.4) (layer "F.Cu") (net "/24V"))
 (segment (start 155.5 78.66) (end 154 77.16) (width 0.4) (layer "F.Cu") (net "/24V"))
 (segment (start 146.5 104.736852) (end 146.5 104.775) (width 0.4) (layer "B.Cu") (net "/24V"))
 (segment (start 146.5 104.736852) (end 146.5 105) (width 0.4) (layer "B.Cu") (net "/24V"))
 (segment (start 144.41 116) (end 143.956 116.454) (width 0.2) (layer "B.Cu") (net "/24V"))
 (segment (start 139.861292 103.85) (end 145.613148 103.85) (width 0.4) (layer "B.Cu") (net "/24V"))
 (segment (start 137.5 104.5) (end 137.5 115.5) (width 0.4) (layer "B.Cu") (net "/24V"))
 (segment (start 146.5 104.5) (end 146.5 105) (width 0.2) (layer "B.Cu") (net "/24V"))
 (segment (start 138.05 103.95) (end 137.5 104.5) (width 0.4) (layer "B.Cu") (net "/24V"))
 (segment (start 147.06 104.44) (end 155.06 104.44) (width 0.4) (layer "B.Cu") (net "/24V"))
 (segment (start 155.06 104.44) (end 155.25 104.25) (width 0.4) (layer "B.Cu") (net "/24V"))
 (segment (start 146.5 104.775) (end 146.5 105) (width 0.2) (layer "B.Cu") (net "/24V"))
 (segment (start 143.524 116.886) (end 144.41 116) (width 0.4) (layer "B.Cu") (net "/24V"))
 (segment (start 139.761292 103.95) (end 139.861292 103.85) (width 0.4) (layer "B.Cu") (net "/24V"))
 (segment (start 137.5 115.5) (end 138.886 116.886) (width 0.4) (layer "B.Cu") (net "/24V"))
 (segment (start 145.613148 103.85) (end 146.5 104.736852) (width 0.4) (layer "B.Cu") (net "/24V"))
 (segment (start 155.25 83.49) (end 154 82.24) (width 0.4) (layer "B.Cu") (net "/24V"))
 (segment (start 146.5 105) (end 147.06 104.44) (width 0.4) (layer "B.Cu") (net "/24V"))
 (segment (start 138.05 103.95) (end 139.761292 103.95) (width 0.4) (layer "B.Cu") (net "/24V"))
 (segment (start 155.25 104.25) (end 155.25 83.49) (width 0.4) (layer "B.Cu") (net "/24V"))
 (segment (start 138.886 116.886) (end 143.524 116.886) (width 0.4) (layer "B.Cu") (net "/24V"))
 (segment (start 154.024999 98) (end 153 98) (width 0.2) (layer "F.Cu") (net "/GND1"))
 (segment (start 145.23 104.775) (end 145.23 105) (width 0.2) (layer "F.Cu") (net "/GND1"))
 (segment (start 156.8 95.224999) (end 154.024999 98) (width 0.2) (layer "F.Cu") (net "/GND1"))
 (segment (start 144.41 118.54) (end 143.135 117.265) (width 0.2) (layer "F.Cu") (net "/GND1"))
 (segment (start 152.005 98) (end 145.23 104.775) (width 0.2) (layer "F.Cu") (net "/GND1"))
 (segment (start 145.23 105.95) (end 145.23 105) (width 0.2) (layer "F.Cu") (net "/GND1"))
 (segment (start 153 98) (end 152.005 98) (width 0.2) (layer "F.Cu") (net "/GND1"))
 (segment (start 143.135 117.265) (end 143.135 108.045) (width 0.2) (layer "F.Cu") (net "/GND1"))
 (segment (start 154 69.54) (end 156.8 72.34) (width 0.2) (layer "F.Cu") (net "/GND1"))
 (segment (start 143.135 108.045) (end 145.23 105.95) (width 0.2) (layer "F.Cu") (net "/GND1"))
 (segment (start 156.8 72.34) (end 156.8 95.224999) (width 0.2) (layer "F.Cu") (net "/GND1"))
 (segment (start 144.5 78.5) (end 150.8 78.5) (width 0.2) (layer "B.Cu") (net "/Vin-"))
 (segment (start 152 79.7) (end 154 79.7) (width 0.2) (layer "B.Cu") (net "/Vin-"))
 (segment (start 150.8 78.5) (end 152 79.7) (width 0.2) (layer "B.Cu") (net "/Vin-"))
 (segment (start 156.4 74.48) (end 156.4 93.084998) (width 0.2) (layer "F.Cu") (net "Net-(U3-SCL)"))
 (segment (start 156.05 93.434999) (end 155.992499 93.492499) (width 0.2) (layer "F.Cu") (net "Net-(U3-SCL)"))
 (segment (start 155.992499 93.492499) (end 154.024999 95.46) (width 0.2) (layer "F.Cu") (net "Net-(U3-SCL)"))
 (segment (start 154.024999 95.46) (end 153 95.46) (width 0.2) (layer "F.Cu") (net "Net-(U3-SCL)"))
 (segment (start 156.4 93.084998) (end 155.992499 93.492499) (width 0.2) (layer "F.Cu") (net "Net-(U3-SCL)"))
 (segment (start 154 72.08) (end 156.4 74.48) (width 0.2) (layer "F.Cu") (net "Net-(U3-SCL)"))
 (segment (start 154 74.62) (end 156 76.62) (width 0.2) (layer "F.Cu") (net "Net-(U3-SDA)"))
 (segment (start 154.024999 91.65) (end 153 91.65) (width 0.2) (layer "F.Cu") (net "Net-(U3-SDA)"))
 (segment (start 156 76.62) (end 156 89.674999) (width 0.2) (layer "F.Cu") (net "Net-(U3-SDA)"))
 (segment (start 156 89.674999) (end 154.024999 91.65) (width 0.2) (layer "F.Cu") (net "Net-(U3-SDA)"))
 (segment (start 149.5 67.46) (end 153.54 67.46) (width 0.2) (layer "F.Cu") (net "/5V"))
 (segment (start 151.8 87.91) (end 153 89.11) (width 0.2) (layer "F.Cu") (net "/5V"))
 (segment (start 143.96 105) (end 143.96 102.559314) (width 0.4) (layer "F.Cu") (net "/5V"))
 (segment (start 143.96 102.559314) (end 146.75 99.769314) (width 0.4) (layer "F.Cu") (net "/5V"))
 (segment (start 154 67) (end 151.8 69.2) (width 0.2) (layer "F.Cu") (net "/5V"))
 (segment (start 153.54 67.46) (end 154 67) (width 0.2) (layer "F.Cu") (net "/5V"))
 (segment (start 146.75 94.335) (end 146.9175 94.1675) (width 0.4) (layer "F.Cu") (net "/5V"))
 (segment (start 146.75 99.769314) (end 146.75 94.335) (width 0.4) (layer "F.Cu") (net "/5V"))
 (segment (start 151.975001 89.11) (end 146.9175 94.1675) (width 0.4) (layer "F.Cu") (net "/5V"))
 (segment (start 153 89.11) (end 151.975001 89.11) (width 0.4) (layer "F.Cu") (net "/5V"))
 (segment (start 151.8 69.2) (end 151.8 87.91) (width 0.2) (layer "F.Cu") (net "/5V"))
 (segment (start 143.96 105.121726) (end 143.96 105) (width 0.2) (layer "B.Cu") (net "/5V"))
 (segment (start 137.695 66.725) (end 143.419365 66.725) (width 0.2) (layer "B.Cu") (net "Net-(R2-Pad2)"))
 (segment (start 147.665 68.165) (end 149.5 70) (width 0.2) (layer "B.Cu") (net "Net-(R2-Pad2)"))
 (segment (start 144.859365 68.165) (end 147.665 68.165) (width 0.2) (layer "B.Cu") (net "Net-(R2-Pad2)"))
 (segment (start 143.419365 66.725) (end 144.859365 68.165) (width 0.2) (layer "B.Cu") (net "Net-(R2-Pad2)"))
 (segment (start 145.315 65.315) (end 144.5 64.5) (width 0.2) (layer "B.Cu") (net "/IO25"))
 (segment (start 112.35 67.65) (end 112.35 93.48) (width 0.2) (layer "B.Cu") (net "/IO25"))
 (segment (start 113.5 66.5) (end 112.35 67.65) (width 0.2) (layer "B.Cu") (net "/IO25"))
 (segment (start 145.315 66.725) (end 145.315 65.315) (width 0.2) (layer "B.Cu") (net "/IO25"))
 (segment (start 112.35 93.48) (end 114 95.13) (width 0.2) (layer "B.Cu") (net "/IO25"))
 (segment (start 144.5 64.5) (end 115.5 64.5) (width 0.2) (layer "B.Cu") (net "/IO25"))
 (segment (start 115.5 64.5) (end 113.5 66.5) (width 0.2) (layer "B.Cu") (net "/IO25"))
 (segment (start 141.9 72) (end 141.9 71.97) (width 0.2) (layer "B.Cu") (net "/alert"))
 (segment (start 144.023654 79.65) (end 141.9 77.526346) (width 0.2) (layer "B.Cu") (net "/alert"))
 (segment (start 154 84.78) (end 153.8 84.58) (width 0.2) (layer "B.Cu") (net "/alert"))
 (segment (start 141.9 77.526346) (end 141.9 72) (width 0.2) (layer "B.Cu") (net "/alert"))
 (segment (start 153.8 84.58) (end 152 84.58) (width 0.2) (layer "B.Cu") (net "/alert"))
 (segment (start 139.165 69.265) (end 141.9 72) (width 0.2) (layer "B.Cu") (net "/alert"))
 (segment (start 137.695 69.265) (end 139.165 69.265) (width 0.2) (layer "B.Cu") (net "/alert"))
 (segment (start 152 84.58) (end 147.07 79.65) (width 0.2) (layer "B.Cu") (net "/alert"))
 (segment (start 147.07 79.65) (end 144.023654 79.65) (width 0.2) (layer "B.Cu") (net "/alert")))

